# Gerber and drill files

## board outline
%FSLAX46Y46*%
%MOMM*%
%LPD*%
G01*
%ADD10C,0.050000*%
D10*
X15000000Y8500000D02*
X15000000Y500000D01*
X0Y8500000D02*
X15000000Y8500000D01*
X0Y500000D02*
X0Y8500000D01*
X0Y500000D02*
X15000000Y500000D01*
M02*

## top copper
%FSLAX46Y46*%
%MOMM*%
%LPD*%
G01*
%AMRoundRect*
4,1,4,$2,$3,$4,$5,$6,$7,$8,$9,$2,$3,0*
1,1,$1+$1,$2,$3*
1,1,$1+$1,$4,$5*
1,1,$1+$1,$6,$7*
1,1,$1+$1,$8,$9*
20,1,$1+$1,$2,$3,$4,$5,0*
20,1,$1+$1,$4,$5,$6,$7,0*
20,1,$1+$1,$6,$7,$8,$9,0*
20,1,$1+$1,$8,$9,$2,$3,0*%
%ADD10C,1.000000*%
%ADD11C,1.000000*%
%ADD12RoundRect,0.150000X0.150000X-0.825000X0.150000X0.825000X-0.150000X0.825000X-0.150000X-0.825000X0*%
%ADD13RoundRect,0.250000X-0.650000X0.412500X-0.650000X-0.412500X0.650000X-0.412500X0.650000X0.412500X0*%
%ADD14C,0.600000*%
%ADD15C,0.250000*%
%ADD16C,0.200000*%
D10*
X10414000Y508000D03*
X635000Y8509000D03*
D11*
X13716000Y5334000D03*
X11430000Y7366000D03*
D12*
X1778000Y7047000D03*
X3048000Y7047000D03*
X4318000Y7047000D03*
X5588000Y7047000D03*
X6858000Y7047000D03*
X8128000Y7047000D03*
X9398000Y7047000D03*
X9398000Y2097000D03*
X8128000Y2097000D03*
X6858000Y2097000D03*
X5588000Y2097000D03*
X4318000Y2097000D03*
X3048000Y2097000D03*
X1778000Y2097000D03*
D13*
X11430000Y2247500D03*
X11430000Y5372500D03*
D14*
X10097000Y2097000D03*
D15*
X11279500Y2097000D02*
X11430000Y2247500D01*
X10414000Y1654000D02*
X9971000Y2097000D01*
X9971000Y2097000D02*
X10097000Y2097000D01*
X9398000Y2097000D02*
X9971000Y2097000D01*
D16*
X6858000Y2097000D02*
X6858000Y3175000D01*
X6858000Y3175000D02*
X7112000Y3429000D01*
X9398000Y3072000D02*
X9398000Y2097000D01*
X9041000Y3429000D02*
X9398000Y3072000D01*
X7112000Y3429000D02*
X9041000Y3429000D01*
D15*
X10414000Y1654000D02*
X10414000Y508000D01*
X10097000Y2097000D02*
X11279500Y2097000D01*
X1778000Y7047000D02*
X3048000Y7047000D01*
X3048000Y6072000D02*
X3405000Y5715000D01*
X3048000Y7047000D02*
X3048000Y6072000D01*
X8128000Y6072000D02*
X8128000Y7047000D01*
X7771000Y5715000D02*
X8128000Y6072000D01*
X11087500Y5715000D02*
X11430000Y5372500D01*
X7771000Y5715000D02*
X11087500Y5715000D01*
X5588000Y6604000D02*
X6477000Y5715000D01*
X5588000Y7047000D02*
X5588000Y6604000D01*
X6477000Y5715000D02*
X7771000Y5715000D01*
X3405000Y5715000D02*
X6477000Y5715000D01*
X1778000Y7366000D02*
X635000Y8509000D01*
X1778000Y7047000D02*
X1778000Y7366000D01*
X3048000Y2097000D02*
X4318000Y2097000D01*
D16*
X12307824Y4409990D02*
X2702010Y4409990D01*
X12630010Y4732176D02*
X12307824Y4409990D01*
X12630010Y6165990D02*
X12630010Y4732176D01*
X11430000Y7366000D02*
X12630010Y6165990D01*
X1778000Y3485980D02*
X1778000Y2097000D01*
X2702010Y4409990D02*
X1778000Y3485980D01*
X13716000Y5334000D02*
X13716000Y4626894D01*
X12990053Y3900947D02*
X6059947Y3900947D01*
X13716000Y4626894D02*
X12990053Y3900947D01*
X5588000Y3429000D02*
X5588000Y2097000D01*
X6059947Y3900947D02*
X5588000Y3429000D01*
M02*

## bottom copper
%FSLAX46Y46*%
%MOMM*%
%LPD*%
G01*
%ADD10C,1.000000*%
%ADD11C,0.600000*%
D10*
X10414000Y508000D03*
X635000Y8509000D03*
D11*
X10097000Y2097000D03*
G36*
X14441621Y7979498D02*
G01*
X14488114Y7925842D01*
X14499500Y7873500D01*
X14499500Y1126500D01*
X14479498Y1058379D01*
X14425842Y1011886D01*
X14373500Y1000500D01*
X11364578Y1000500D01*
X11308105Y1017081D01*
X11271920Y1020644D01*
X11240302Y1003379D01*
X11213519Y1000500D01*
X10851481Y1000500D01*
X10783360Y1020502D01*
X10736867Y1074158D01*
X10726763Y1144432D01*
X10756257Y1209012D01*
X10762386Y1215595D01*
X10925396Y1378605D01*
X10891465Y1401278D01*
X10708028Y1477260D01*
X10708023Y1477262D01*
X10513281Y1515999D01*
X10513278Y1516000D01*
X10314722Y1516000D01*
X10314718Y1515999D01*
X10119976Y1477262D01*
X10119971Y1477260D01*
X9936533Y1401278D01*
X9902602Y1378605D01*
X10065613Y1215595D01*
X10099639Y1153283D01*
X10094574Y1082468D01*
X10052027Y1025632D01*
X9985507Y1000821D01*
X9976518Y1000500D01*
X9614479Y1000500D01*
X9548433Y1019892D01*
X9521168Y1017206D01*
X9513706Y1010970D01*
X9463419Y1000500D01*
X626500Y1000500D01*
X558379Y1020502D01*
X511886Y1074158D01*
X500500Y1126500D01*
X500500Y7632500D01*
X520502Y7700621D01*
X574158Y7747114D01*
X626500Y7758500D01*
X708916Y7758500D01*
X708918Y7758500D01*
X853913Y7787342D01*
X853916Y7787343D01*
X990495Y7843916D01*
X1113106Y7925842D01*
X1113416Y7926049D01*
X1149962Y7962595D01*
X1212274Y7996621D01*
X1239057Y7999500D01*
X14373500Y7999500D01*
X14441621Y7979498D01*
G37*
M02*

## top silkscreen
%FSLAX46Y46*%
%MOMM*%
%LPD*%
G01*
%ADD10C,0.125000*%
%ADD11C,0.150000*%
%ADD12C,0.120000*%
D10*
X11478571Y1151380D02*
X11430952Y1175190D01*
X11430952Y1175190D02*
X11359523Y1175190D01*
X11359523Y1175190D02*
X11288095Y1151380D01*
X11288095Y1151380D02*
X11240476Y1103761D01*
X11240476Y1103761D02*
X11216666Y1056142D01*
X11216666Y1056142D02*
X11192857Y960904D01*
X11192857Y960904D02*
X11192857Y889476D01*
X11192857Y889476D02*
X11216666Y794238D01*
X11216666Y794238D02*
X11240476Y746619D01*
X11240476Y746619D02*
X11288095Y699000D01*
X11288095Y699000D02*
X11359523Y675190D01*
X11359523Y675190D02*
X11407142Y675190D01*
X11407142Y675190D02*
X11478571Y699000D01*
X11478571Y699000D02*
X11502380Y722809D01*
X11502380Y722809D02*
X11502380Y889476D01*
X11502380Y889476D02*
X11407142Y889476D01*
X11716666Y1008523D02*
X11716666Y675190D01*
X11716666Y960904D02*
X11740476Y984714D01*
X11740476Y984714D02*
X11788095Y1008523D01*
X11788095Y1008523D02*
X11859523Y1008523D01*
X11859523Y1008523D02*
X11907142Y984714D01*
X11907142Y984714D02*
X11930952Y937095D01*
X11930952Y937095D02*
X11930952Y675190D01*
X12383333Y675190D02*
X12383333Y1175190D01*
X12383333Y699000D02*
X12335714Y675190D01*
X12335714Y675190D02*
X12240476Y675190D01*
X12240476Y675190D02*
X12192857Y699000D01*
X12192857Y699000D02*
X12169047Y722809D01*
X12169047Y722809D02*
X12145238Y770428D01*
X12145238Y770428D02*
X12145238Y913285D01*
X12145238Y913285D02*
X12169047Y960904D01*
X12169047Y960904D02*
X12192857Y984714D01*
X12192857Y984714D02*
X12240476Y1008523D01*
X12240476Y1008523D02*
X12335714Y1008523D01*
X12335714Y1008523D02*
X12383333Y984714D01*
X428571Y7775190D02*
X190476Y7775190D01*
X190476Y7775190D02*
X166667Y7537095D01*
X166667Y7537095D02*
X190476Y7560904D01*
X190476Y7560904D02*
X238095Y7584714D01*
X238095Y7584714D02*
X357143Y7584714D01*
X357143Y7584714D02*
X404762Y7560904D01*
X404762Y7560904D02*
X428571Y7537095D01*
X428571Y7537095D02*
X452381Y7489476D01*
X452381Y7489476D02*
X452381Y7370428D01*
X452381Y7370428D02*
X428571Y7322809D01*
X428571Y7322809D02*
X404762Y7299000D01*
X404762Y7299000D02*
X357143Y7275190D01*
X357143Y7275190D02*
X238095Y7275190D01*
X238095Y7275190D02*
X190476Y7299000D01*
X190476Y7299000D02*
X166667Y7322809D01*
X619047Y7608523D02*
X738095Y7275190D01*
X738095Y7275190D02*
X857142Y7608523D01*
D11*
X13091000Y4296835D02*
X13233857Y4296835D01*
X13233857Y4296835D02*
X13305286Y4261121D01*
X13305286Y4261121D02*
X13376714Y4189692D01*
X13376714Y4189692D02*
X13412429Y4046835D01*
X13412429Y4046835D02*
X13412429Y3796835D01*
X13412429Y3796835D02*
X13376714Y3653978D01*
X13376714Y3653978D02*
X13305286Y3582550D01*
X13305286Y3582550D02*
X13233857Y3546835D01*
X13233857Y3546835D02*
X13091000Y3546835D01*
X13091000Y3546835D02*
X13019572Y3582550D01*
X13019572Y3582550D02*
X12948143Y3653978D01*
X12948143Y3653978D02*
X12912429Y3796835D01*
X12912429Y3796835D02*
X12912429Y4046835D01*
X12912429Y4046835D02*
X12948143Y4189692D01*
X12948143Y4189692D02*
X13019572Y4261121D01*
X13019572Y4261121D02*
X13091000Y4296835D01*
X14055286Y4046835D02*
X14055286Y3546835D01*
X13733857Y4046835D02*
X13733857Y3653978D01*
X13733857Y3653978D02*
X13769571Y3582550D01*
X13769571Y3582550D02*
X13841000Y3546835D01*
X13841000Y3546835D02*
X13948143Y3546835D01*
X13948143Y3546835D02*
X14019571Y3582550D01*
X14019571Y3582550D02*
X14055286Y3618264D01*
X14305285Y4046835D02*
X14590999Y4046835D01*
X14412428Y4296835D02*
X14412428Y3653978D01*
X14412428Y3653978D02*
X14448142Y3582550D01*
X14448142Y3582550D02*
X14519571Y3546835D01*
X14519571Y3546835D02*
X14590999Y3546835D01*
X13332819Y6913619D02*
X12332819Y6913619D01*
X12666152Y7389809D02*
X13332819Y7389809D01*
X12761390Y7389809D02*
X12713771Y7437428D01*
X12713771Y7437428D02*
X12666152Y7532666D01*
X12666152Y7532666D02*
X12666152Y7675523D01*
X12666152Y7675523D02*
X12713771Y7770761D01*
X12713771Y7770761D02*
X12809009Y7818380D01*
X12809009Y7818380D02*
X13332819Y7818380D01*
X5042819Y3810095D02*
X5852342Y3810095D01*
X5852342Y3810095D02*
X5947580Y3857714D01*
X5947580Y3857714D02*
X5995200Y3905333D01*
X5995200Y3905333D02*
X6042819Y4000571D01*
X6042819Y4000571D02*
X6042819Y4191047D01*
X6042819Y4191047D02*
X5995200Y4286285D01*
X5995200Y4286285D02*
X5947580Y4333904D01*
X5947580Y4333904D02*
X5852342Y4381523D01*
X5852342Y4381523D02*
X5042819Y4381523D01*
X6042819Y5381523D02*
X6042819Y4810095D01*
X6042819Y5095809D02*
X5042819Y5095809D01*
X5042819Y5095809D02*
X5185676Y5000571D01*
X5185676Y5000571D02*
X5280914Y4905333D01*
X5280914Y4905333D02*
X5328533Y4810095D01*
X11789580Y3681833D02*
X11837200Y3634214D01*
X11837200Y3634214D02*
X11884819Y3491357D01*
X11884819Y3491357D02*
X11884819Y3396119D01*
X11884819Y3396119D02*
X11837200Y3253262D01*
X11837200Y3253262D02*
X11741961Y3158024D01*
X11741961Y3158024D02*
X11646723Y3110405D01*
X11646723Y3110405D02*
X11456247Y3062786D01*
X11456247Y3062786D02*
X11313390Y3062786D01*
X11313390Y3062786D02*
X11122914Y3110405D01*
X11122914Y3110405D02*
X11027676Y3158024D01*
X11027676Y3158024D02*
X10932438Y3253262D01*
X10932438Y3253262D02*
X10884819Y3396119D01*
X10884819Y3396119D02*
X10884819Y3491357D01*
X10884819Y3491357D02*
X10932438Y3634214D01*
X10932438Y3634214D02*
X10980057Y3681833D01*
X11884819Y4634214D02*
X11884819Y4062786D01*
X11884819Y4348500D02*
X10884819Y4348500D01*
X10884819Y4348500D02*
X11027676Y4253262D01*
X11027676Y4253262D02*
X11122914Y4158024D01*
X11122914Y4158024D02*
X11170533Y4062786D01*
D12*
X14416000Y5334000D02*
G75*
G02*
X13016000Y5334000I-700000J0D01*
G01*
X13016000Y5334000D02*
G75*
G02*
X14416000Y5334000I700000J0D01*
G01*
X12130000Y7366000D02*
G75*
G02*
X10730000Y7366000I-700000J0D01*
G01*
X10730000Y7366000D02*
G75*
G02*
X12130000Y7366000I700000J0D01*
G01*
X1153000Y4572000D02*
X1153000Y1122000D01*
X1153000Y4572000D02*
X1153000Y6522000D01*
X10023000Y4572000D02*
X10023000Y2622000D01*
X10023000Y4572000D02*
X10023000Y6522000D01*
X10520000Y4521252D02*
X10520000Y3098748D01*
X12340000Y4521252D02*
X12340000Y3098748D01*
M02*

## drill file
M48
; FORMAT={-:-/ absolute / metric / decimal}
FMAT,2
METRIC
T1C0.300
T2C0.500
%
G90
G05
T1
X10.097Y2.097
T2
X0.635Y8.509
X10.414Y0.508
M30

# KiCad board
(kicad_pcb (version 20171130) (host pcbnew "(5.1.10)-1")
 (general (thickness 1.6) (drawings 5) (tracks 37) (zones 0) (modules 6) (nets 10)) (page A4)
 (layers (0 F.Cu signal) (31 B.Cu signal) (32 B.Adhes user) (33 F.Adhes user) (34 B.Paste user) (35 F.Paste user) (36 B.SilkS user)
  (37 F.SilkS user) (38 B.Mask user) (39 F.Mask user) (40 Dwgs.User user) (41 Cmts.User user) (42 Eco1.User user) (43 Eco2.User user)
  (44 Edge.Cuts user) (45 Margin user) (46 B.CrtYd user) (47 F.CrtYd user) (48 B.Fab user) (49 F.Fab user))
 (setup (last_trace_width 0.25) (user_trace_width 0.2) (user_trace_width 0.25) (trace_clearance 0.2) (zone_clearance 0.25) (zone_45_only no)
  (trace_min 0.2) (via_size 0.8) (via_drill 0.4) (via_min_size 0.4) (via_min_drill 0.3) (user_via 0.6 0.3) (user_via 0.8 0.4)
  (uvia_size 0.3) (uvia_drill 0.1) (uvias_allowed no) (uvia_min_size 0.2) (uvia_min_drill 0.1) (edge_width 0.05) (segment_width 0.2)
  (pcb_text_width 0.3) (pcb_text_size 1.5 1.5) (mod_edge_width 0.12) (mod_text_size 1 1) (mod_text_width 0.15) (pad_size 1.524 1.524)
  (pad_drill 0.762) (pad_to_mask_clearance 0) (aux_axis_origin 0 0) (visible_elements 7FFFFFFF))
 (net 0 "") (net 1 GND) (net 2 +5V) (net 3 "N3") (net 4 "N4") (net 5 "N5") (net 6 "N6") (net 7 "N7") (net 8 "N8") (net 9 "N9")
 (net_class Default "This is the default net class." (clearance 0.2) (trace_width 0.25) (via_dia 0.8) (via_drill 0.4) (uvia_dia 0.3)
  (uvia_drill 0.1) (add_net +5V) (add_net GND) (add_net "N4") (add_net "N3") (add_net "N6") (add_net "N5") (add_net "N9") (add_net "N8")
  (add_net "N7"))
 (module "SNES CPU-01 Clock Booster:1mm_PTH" (layer F.Cu) (at 10.414 -0.508)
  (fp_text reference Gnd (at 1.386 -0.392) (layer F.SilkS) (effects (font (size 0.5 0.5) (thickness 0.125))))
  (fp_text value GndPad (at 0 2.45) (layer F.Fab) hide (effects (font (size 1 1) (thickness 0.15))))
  (pad 1 thru_hole circle (at 0 0) (size 1 1) (drill 0.5) (layers *.Cu *.Mask) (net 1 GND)))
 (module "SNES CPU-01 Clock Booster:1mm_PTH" (layer F.Cu) (at 0.635 -8.509)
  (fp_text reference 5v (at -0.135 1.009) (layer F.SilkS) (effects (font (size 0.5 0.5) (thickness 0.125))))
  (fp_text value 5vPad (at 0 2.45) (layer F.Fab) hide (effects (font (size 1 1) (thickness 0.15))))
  (pad 1 thru_hole circle (at 0 0) (size 1 1) (drill 0.5) (layers *.Cu *.Mask) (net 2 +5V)))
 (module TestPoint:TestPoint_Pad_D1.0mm (layer F.Cu) (at 13.716 -5.334 180)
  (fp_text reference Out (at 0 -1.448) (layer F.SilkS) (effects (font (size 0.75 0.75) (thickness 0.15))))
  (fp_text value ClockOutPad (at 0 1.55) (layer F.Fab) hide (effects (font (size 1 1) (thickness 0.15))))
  (fp_circle (center 0 0) (end 0 0.7) (layer F.SilkS) (width 0.12))
  (pad 1 smd circle (at 0 0 180) (size 1 1) (layers F.Cu F.Mask) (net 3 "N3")))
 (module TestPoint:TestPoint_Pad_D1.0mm (layer F.Cu) (at 11.43 -7.366 270)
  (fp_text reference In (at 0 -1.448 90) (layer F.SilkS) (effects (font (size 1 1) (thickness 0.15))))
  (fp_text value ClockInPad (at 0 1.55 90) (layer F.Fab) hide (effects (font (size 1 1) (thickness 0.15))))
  (fp_circle (center 0 0) (end 0 0.7) (layer F.SilkS) (width 0.12))
  (pad 1 smd circle (at 0 0 270) (size 1 1) (layers F.Cu F.Mask) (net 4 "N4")))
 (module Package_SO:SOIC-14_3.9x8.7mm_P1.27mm (layer F.Cu) (at 5.588 -4.572 90)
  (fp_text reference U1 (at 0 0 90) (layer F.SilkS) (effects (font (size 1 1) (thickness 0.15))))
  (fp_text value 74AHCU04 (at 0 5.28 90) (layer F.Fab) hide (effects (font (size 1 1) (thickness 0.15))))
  (fp_line (start 0 -4.435) (end -3.45 -4.435) (layer F.SilkS) (width 0.12))
  (fp_line (start 0 -4.435) (end 1.95 -4.435) (layer F.SilkS) (width 0.12))
  (fp_line (start 0 4.435) (end -1.95 4.435) (layer F.SilkS) (width 0.12))
  (fp_line (start 0 4.435) (end 1.95 4.435) (layer F.SilkS) (width 0.12))
  (pad 14 smd roundrect (at 2.475 -3.81 90) (size 1.95 0.6) (layers F.Cu F.Paste F.Mask) (roundrect_rratio 0.25) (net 2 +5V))
  (pad 13 smd roundrect (at 2.475 -2.54 90) (size 1.95 0.6) (layers F.Cu F.Paste F.Mask) (roundrect_rratio 0.25) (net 2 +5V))
  (pad 12 smd roundrect (at 2.475 -1.27 90) (size 1.95 0.6) (layers F.Cu F.Paste F.Mask) (roundrect_rratio 0.25) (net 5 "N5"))
  (pad 11 smd roundrect (at 2.475 0 90) (size 1.95 0.6) (layers F.Cu F.Paste F.Mask) (roundrect_rratio 0.25) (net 2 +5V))
  (pad 10 smd roundrect (at 2.475 1.27 90) (size 1.95 0.6) (layers F.Cu F.Paste F.Mask) (roundrect_rratio 0.25) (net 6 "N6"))
  (pad 9 smd roundrect (at 2.475 2.54 90) (size 1.95 0.6) (layers F.Cu F.Paste F.Mask) (roundrect_rratio 0.25) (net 2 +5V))
  (pad 8 smd roundrect (at 2.475 3.81 90) (size 1.95 0.6) (layers F.Cu F.Paste F.Mask) (roundrect_rratio 0.25) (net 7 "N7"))
  (pad 7 smd roundrect (at -2.475 3.81 90) (size 1.95 0.6) (layers F.Cu F.Paste F.Mask) (roundrect_rratio 0.25) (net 1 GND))
  (pad 6 smd roundrect (at -2.475 2.54 90) (size 1.95 0.6) (layers F.Cu F.Paste F.Mask) (roundrect_rratio 0.25) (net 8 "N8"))
  (pad 5 smd roundrect (at -2.475 1.27 90) (size 1.95 0.6) (layers F.Cu F.Paste F.Mask) (roundrect_rratio 0.25) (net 1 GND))
  (pad 4 smd roundrect (at -2.475 0 90) (size 1.95 0.6) (layers F.Cu F.Paste F.Mask) (roundrect_rratio 0.25) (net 3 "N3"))
  (pad 3 smd roundrect (at -2.475 -1.27 90) (size 1.95 0.6) (layers F.Cu F.Paste F.Mask) (roundrect_rratio 0.25) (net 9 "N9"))
  (pad 2 smd roundrect (at -2.475 -2.54 90) (size 1.95 0.6) (layers F.Cu F.Paste F.Mask) (roundrect_rratio 0.25) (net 9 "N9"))
  (pad 1 smd roundrect (at -2.475 -3.81 90) (size 1.95 0.6) (layers F.Cu F.Paste F.Mask) (roundrect_rratio 0.25) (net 4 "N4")))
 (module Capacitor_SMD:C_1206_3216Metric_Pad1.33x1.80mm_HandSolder (layer F.Cu) (at 11.43 -3.81 270)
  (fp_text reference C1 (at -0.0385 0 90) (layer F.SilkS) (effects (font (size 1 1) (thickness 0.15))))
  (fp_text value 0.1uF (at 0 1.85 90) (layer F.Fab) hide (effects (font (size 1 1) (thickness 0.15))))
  (fp_line (start -0.711252 0.91) (end 0.711252 0.91) (layer F.SilkS) (width 0.12))
  (fp_line (start -0.711252 -0.91) (end 0.711252 -0.91) (layer F.SilkS) (width 0.12))
  (pad 2 smd roundrect (at 1.5625 0 270) (size 1.325 1.8) (layers F.Cu F.Paste F.Mask) (roundrect_rratio 0.188679) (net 1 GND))
  (pad 1 smd roundrect (at -1.5625 0 270) (size 1.325 1.8) (layers F.Cu F.Paste F.Mask) (roundrect_rratio 0.188679) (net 2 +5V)))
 (gr_line (start 15 -8.5) (end 15 -0.5) (layer Edge.Cuts) (width 0.05))
 (gr_line (start 0 -8.5) (end 15 -8.5) (layer Edge.Cuts) (width 0.05))
 (gr_line (start 0 -0.5) (end 0 -8.5) (layer Edge.Cuts) (width 0.05))
 (gr_line (start 0 -0.5) (end 15 -0.5) (layer Edge.Cuts) (width 0.05))
 (segment (start 11.2795 -2.097) (end 11.43 -2.2475) (width 0.25) (layer F.Cu) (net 1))
 (segment (start 10.414 -1.654) (end 9.971 -2.097) (width 0.25) (layer F.Cu) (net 1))
 (segment (start 9.971 -2.097) (end 10.097 -2.097) (width 0.25) (layer F.Cu) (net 1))
 (segment (start 9.398 -2.097) (end 9.971 -2.097) (width 0.25) (layer F.Cu) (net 1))
 (segment (start 6.858 -2.097) (end 6.858 -3.175) (width 0.2) (layer F.Cu) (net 1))
 (segment (start 6.858 -3.175) (end 7.112 -3.429) (width 0.2) (layer F.Cu) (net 1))
 (segment (start 9.398 -3.072) (end 9.398 -2.097) (width 0.2) (layer F.Cu) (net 1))
 (segment (start 9.041 -3.429) (end 9.398 -3.072) (width 0.2) (layer F.Cu) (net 1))
 (segment (start 7.112 -3.429) (end 9.041 -3.429) (width 0.2) (layer F.Cu) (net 1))
 (segment (start 10.414 -1.654) (end 10.414 -0.508) (width 0.25) (layer F.Cu) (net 1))
 (segment (start 10.097 -2.097) (end 11.2795 -2.097) (width 0.25) (layer F.Cu) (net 1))
 (via (at 10.097 -2.097) (size 0.6) (drill 0.3) (layers F.Cu B.Cu) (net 1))
 (segment (start 1.778 -7.047) (end 3.048 -7.047) (width 0.25) (layer F.Cu) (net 2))
 (segment (start 3.048 -6.072) (end 3.405 -5.715) (width 0.25) (layer F.Cu) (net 2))
 (segment (start 3.048 -7.047) (end 3.048 -6.072) (width 0.25) (layer F.Cu) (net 2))
 (segment (start 8.128 -6.072) (end 8.128 -7.047) (width 0.25) (layer F.Cu) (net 2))
 (segment (start 7.771 -5.715) (end 8.128 -6.072) (width 0.25) (layer F.Cu) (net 2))
 (segment (start 11.0875 -5.715) (end 11.43 -5.3725) (width 0.25) (layer F.Cu) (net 2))
 (segment (start 7.771 -5.715) (end 11.0875 -5.715) (width 0.25) (layer F.Cu) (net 2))
 (segment (start 5.588 -6.604) (end 6.477 -5.715) (width 0.25) (layer F.Cu) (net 2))
 (segment (start 5.588 -7.047) (end 5.588 -6.604) (width 0.25) (layer F.Cu) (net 2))
 (segment (start 6.477 -5.715) (end 7.771 -5.715) (width 0.25) (layer F.Cu) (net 2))
 (segment (start 3.405 -5.715) (end 6.477 -5.715) (width 0.25) (layer F.Cu) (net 2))
 (segment (start 1.778 -7.366) (end 0.635 -8.509) (width 0.25) (layer F.Cu) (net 2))
 (segment (start 1.778 -7.047) (end 1.778 -7.366) (width 0.25) (layer F.Cu) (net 2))
 (segment (start 3.048 -2.097) (end 4.318 -2.097) (width 0.25) (layer F.Cu) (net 9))
 (segment (start 12.307824 -4.40999) (end 2.70201 -4.40999) (width 0.2) (layer F.Cu) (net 4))
 (segment (start 12.63001 -4.732176) (end 12.307824 -4.40999) (width 0.2) (layer F.Cu) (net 4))
 (segment (start 12.63001 -6.16599) (end 12.63001 -4.732176) (width 0.2) (layer F.Cu) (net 4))
 (segment (start 11.43 -7.366) (end 12.63001 -6.16599) (width 0.2) (layer F.Cu) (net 4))
 (segment (start 1.778 -3.48598) (end 1.778 -2.097) (width 0.2) (layer F.Cu) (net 4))
 (segment (start 2.70201 -4.40999) (end 1.778 -3.48598) (width 0.2) (layer F.Cu) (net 4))
 (segment (start 13.716 -5.334) (end 13.716 -4.626894) (width 0.2) (layer F.Cu) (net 3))
 (segment (start 12.990053 -3.900947) (end 6.059947 -3.900947) (width 0.2) (layer F.Cu) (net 3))
 (segment (start 13.716 -4.626894) (end 12.990053 -3.900947) (width 0.2) (layer F.Cu) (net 3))
 (segment (start 5.588 -3.429) (end 5.588 -2.097) (width 0.2) (layer F.Cu) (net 3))
 (segment (start 6.059947 -3.900947) (end 5.588 -3.429) (width 0.2) (layer F.Cu) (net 3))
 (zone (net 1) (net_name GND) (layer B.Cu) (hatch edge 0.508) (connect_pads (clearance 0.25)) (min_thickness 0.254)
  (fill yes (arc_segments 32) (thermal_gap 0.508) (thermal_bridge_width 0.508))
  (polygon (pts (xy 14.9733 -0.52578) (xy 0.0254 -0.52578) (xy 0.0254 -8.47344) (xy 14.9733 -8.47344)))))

